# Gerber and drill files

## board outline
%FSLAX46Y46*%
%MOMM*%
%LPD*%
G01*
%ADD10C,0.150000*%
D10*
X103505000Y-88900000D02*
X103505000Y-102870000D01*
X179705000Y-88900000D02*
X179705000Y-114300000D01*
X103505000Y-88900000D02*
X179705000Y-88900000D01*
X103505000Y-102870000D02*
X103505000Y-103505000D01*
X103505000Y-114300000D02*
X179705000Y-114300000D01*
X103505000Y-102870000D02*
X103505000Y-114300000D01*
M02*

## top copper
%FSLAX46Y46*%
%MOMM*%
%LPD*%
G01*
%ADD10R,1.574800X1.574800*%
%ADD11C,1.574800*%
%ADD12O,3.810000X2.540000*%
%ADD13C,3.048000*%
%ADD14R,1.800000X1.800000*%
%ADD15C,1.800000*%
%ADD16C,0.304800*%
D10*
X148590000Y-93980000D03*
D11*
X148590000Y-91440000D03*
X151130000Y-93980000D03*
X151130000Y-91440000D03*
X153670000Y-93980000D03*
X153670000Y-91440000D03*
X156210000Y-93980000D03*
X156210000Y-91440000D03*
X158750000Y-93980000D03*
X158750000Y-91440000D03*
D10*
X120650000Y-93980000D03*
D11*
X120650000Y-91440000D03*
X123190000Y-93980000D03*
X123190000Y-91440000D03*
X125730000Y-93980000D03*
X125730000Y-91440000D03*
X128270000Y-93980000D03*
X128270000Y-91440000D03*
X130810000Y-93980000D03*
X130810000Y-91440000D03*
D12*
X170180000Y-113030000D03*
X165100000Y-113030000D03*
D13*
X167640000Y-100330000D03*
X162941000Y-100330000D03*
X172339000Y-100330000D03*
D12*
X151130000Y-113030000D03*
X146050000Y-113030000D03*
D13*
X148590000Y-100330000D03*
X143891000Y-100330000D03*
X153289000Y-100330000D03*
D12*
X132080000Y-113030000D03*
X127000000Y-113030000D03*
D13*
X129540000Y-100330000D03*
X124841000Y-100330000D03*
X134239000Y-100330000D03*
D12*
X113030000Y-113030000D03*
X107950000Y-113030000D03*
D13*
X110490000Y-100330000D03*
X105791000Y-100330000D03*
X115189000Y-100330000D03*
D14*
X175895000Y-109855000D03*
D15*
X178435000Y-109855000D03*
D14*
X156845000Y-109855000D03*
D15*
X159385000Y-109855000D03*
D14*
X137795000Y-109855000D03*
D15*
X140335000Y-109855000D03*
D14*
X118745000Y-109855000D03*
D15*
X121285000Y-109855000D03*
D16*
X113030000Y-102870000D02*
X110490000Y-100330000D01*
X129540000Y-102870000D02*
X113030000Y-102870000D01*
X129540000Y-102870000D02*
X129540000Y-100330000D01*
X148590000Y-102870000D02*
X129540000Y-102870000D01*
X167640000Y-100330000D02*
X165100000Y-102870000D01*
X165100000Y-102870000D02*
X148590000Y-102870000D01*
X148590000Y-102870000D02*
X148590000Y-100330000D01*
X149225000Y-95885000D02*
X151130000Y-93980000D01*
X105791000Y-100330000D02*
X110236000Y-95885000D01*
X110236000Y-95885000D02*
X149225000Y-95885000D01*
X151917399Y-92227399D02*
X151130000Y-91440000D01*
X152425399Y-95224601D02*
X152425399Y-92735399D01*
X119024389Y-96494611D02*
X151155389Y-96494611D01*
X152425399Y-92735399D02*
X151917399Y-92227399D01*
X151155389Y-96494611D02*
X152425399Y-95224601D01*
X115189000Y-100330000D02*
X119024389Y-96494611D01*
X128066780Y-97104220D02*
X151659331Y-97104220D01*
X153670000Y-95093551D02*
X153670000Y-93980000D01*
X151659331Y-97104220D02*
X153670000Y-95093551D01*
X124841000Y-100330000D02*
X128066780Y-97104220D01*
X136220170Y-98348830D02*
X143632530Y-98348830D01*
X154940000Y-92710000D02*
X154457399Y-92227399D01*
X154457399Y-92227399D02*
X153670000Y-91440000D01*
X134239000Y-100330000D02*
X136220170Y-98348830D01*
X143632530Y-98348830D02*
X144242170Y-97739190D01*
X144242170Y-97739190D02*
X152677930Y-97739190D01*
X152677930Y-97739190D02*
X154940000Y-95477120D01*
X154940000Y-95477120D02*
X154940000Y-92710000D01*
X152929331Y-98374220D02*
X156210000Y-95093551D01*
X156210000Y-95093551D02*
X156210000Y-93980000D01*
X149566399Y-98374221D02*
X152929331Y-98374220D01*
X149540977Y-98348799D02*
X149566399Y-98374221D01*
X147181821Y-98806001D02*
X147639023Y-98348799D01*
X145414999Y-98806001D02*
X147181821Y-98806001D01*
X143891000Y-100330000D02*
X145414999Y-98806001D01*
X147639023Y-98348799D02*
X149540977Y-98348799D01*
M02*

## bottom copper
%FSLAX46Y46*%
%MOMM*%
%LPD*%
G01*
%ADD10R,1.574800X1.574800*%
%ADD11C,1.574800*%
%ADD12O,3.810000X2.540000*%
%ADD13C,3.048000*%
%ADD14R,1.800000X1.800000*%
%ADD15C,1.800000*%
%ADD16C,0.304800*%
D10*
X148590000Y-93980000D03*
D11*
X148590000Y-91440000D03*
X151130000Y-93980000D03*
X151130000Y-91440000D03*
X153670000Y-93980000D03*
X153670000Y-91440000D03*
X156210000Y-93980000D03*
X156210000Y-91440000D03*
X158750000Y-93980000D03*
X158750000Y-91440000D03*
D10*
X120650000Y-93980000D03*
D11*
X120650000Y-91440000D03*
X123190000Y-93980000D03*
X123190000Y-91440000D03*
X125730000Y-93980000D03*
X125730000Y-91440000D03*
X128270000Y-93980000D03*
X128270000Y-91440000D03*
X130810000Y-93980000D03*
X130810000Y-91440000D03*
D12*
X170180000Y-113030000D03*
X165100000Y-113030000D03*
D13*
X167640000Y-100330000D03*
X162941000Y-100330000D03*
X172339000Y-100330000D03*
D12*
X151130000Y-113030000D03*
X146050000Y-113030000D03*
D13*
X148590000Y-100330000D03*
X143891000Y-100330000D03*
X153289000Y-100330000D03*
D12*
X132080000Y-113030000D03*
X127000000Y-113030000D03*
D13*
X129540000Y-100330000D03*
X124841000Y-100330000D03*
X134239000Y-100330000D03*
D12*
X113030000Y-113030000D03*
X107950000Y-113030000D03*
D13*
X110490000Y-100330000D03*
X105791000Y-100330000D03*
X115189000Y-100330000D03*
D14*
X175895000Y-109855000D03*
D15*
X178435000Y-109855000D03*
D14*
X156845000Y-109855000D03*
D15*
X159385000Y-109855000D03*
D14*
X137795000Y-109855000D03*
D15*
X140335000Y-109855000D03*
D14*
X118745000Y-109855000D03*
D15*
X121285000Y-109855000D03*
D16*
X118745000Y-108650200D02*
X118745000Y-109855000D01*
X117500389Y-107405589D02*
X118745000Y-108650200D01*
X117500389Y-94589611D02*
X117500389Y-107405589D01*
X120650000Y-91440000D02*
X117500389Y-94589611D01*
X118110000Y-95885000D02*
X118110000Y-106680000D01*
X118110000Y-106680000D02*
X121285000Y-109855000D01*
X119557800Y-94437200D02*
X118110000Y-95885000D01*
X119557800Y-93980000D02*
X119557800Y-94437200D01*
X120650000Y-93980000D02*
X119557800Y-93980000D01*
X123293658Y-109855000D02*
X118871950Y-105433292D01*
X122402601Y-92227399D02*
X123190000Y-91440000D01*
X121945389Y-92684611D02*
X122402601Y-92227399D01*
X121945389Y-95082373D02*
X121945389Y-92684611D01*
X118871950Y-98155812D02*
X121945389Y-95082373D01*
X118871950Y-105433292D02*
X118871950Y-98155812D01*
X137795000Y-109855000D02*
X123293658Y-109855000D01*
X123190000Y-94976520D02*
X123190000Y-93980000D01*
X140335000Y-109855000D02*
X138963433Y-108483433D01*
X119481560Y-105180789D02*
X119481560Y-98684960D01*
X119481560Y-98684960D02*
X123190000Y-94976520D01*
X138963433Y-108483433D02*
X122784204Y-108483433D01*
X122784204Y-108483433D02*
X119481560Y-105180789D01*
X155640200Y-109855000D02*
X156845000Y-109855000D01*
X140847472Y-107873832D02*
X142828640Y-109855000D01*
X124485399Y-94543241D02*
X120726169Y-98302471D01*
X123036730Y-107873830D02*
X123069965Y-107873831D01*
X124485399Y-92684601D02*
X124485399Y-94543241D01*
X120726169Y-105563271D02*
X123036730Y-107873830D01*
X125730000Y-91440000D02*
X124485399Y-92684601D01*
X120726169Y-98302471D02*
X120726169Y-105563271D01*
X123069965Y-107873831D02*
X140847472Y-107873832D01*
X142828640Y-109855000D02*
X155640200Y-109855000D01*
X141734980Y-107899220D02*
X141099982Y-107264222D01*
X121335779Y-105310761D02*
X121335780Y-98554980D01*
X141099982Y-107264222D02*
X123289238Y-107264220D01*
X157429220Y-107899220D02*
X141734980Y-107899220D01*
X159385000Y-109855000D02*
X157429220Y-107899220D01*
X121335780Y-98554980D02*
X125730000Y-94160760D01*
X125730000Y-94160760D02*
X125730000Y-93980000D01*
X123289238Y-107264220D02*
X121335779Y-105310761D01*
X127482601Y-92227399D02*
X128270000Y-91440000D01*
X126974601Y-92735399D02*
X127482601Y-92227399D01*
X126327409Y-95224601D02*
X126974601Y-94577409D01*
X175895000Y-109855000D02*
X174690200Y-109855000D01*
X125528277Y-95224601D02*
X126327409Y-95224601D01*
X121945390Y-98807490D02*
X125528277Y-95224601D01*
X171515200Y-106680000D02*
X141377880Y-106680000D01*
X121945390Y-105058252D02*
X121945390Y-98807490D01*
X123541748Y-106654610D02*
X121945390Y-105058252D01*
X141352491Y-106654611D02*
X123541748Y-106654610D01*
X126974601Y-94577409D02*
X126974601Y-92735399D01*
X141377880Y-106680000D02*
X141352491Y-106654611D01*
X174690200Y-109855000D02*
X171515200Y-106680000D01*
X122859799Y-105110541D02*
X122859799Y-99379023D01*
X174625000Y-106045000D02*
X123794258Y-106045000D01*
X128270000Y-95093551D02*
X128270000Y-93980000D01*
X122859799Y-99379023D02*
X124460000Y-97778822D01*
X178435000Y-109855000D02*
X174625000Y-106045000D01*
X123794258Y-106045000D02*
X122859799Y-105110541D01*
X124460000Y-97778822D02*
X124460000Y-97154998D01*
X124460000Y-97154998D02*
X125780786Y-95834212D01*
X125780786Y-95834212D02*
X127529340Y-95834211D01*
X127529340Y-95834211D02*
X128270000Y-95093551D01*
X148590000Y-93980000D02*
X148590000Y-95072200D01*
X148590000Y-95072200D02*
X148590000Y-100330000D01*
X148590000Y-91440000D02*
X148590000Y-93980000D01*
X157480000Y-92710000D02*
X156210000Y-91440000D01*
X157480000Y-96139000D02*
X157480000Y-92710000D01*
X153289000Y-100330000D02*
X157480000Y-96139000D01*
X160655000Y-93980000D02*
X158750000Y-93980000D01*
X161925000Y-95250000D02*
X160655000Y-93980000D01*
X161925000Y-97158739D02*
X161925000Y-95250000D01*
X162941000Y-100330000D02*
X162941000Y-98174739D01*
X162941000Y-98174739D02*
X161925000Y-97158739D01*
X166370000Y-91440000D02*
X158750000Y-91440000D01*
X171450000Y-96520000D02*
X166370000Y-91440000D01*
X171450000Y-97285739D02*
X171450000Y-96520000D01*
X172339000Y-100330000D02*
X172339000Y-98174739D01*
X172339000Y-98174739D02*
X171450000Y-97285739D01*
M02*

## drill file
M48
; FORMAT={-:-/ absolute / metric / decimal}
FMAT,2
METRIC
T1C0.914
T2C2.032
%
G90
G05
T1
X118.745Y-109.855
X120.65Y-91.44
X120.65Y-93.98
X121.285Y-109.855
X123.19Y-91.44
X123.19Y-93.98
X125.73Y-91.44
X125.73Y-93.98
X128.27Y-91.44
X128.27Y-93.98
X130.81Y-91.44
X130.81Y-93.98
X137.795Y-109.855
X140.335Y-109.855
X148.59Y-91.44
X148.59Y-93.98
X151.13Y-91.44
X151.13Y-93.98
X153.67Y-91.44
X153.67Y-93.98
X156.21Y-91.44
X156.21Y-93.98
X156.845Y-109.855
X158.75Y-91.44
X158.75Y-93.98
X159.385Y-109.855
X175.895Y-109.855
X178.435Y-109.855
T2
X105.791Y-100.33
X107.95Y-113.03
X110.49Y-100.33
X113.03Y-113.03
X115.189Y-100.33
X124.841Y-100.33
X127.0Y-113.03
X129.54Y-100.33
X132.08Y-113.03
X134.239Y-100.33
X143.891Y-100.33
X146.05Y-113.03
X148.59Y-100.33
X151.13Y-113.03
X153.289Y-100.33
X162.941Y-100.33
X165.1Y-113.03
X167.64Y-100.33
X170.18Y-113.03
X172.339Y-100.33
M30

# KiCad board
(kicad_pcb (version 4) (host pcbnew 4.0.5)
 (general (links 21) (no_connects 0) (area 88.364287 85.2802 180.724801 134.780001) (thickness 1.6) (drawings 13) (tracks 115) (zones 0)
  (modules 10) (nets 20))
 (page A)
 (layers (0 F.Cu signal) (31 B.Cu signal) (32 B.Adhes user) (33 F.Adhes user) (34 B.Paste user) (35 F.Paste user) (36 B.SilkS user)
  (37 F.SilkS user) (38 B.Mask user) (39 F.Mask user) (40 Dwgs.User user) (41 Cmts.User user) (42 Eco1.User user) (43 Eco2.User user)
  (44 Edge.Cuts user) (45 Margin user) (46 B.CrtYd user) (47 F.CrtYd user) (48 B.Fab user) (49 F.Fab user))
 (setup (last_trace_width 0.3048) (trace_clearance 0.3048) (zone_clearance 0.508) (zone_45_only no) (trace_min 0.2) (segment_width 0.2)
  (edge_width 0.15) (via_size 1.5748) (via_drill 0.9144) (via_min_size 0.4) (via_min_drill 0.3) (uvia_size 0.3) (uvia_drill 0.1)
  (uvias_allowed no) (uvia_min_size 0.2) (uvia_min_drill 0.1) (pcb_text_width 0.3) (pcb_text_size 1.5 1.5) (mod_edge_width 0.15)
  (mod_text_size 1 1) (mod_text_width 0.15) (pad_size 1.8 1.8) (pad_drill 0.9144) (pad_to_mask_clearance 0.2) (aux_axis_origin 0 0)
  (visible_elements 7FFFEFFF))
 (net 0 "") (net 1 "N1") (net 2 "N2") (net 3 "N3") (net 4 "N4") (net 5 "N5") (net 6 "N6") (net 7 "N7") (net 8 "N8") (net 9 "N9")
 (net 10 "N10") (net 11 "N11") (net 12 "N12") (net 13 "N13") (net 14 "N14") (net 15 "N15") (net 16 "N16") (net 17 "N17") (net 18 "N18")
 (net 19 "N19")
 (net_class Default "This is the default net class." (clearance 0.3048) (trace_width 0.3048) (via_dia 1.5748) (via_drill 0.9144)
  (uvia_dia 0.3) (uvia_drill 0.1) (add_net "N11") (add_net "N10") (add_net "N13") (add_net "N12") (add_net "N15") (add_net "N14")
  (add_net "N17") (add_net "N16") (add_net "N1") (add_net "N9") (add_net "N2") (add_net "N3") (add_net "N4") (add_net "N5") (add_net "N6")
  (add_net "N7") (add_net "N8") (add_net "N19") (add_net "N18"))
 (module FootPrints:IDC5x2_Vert (layer F.Cu) (at 153.67 92.71 180)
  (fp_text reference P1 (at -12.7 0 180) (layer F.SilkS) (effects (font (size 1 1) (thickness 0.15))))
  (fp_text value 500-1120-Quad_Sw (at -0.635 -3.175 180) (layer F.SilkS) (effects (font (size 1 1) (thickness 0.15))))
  (pad 1 thru_hole rect (at 5.08 -1.27 180) (size 1.5748 1.5748) (drill 0.9144) (layers *.Cu *.Mask F.SilkS) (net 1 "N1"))
  (pad 2 thru_hole circle (at 5.08 1.27 180) (size 1.5748 1.5748) (drill 0.9144) (layers *.Cu *.Mask F.SilkS) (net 1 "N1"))
  (pad 3 thru_hole circle (at 2.54 -1.27 180) (size 1.5748 1.5748) (drill 0.9144) (layers *.Cu *.Mask F.SilkS) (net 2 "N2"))
  (pad 4 thru_hole circle (at 2.54 1.27 180) (size 1.5748 1.5748) (drill 0.9144) (layers *.Cu *.Mask F.SilkS) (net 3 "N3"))
  (pad 5 thru_hole circle (at 0 -1.27 180) (size 1.5748 1.5748) (drill 0.9144) (layers *.Cu *.Mask F.SilkS) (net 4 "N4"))
  (pad 6 thru_hole circle (at 0 1.27 180) (size 1.5748 1.5748) (drill 0.9144) (layers *.Cu *.Mask F.SilkS) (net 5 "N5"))
  (pad 7 thru_hole circle (at -2.54 -1.27 180) (size 1.5748 1.5748) (drill 0.9144) (layers *.Cu *.Mask F.SilkS) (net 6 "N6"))
  (pad 8 thru_hole circle (at -2.54 1.27 180) (size 1.5748 1.5748) (drill 0.9144) (layers *.Cu *.Mask F.SilkS) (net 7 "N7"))
  (pad 9 thru_hole circle (at -5.08 -1.27 180) (size 1.5748 1.5748) (drill 0.9144) (layers *.Cu *.Mask F.SilkS) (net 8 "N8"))
  (pad 10 thru_hole circle (at -5.08 1.27 180) (size 1.5748 1.5748) (drill 0.9144) (layers *.Cu *.Mask F.SilkS) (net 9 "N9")))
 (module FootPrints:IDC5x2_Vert (layer F.Cu) (at 125.73 92.71 180)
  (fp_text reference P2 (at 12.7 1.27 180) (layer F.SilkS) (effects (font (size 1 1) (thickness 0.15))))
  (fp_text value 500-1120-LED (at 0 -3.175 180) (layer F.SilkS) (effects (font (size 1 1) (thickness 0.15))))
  (pad 1 thru_hole rect (at 5.08 -1.27 180) (size 1.5748 1.5748) (drill 0.9144) (layers *.Cu *.Mask F.SilkS) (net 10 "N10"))
  (pad 2 thru_hole circle (at 5.08 1.27 180) (size 1.5748 1.5748) (drill 0.9144) (layers *.Cu *.Mask F.SilkS) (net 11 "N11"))
  (pad 3 thru_hole circle (at 2.54 -1.27 180) (size 1.5748 1.5748) (drill 0.9144) (layers *.Cu *.Mask F.SilkS) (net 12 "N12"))
  (pad 4 thru_hole circle (at 2.54 1.27 180) (size 1.5748 1.5748) (drill 0.9144) (layers *.Cu *.Mask F.SilkS) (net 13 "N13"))
  (pad 5 thru_hole circle (at 0 -1.27 180) (size 1.5748 1.5748) (drill 0.9144) (layers *.Cu *.Mask F.SilkS) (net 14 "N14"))
  (pad 6 thru_hole circle (at 0 1.27 180) (size 1.5748 1.5748) (drill 0.9144) (layers *.Cu *.Mask F.SilkS) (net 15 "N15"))
  (pad 7 thru_hole circle (at -2.54 -1.27 180) (size 1.5748 1.5748) (drill 0.9144) (layers *.Cu *.Mask F.SilkS) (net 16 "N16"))
  (pad 8 thru_hole circle (at -2.54 1.27 180) (size 1.5748 1.5748) (drill 0.9144) (layers *.Cu *.Mask F.SilkS) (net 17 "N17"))
  (pad 9 thru_hole circle (at -5.08 -1.27 180) (size 1.5748 1.5748) (drill 0.9144) (layers *.Cu *.Mask F.SilkS) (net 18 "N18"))
  (pad 10 thru_hole circle (at -5.08 1.27 180) (size 1.5748 1.5748) (drill 0.9144) (layers *.Cu *.Mask F.SilkS) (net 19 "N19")))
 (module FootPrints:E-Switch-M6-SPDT (layer F.Cu) (at 167.64 113.03 180)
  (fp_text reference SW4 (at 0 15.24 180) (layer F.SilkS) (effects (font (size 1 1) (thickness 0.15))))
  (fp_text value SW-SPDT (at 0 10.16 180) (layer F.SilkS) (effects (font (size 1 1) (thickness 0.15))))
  (pad 4 thru_hole oval (at -2.54 0 180) (size 3.81 2.54) (drill 2.032) (layers *.Cu *.Mask))
  (pad 5 thru_hole oval (at 2.54 0 180) (size 3.81 2.54) (drill 2.032) (layers *.Cu *.Mask))
  (pad 2 thru_hole circle (at 0 12.7 180) (size 3.048 3.048) (drill 2.032) (layers *.Cu *.Mask) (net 1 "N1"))
  (pad 3 thru_hole circle (at 4.699 12.7 180) (size 3.048 3.048) (drill 2.032) (layers *.Cu *.Mask) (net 8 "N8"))
  (pad 1 thru_hole circle (at -4.699 12.7 180) (size 3.048 3.048) (drill 2.032) (layers *.Cu *.Mask) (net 9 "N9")))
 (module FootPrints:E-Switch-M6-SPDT (layer F.Cu) (at 148.59 113.03 180)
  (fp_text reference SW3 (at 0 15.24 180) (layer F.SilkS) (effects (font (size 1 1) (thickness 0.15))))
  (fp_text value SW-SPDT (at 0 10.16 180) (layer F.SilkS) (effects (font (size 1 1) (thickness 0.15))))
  (pad 4 thru_hole oval (at -2.54 0 180) (size 3.81 2.54) (drill 2.032) (layers *.Cu *.Mask))
  (pad 5 thru_hole oval (at 2.54 0 180) (size 3.81 2.54) (drill 2.032) (layers *.Cu *.Mask))
  (pad 2 thru_hole circle (at 0 12.7 180) (size 3.048 3.048) (drill 2.032) (layers *.Cu *.Mask) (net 1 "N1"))
  (pad 3 thru_hole circle (at 4.699 12.7 180) (size 3.048 3.048) (drill 2.032) (layers *.Cu *.Mask) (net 6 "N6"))
  (pad 1 thru_hole circle (at -4.699 12.7 180) (size 3.048 3.048) (drill 2.032) (layers *.Cu *.Mask) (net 7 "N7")))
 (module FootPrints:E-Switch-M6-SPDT (layer F.Cu) (at 129.54 113.03 180)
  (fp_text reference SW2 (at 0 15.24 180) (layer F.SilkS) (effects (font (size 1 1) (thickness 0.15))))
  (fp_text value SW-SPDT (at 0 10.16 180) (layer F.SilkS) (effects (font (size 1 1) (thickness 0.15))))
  (pad 4 thru_hole oval (at -2.54 0 180) (size 3.81 2.54) (drill 2.032) (layers *.Cu *.Mask))
  (pad 5 thru_hole oval (at 2.54 0 180) (size 3.81 2.54) (drill 2.032) (layers *.Cu *.Mask))
  (pad 2 thru_hole circle (at 0 12.7 180) (size 3.048 3.048) (drill 2.032) (layers *.Cu *.Mask) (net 1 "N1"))
  (pad 3 thru_hole circle (at 4.699 12.7 180) (size 3.048 3.048) (drill 2.032) (layers *.Cu *.Mask) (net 4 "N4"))
  (pad 1 thru_hole circle (at -4.699 12.7 180) (size 3.048 3.048) (drill 2.032) (layers *.Cu *.Mask) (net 5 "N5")))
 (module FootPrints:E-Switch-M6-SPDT (layer F.Cu) (at 110.49 113.03 180)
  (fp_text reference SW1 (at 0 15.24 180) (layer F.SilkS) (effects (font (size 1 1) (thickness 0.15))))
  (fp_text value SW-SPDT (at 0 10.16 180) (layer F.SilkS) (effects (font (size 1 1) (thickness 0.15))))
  (pad 4 thru_hole oval (at -2.54 0 180) (size 3.81 2.54) (drill 2.032) (layers *.Cu *.Mask))
  (pad 5 thru_hole oval (at 2.54 0 180) (size 3.81 2.54) (drill 2.032) (layers *.Cu *.Mask))
  (pad 2 thru_hole circle (at 0 12.7 180) (size 3.048 3.048) (drill 2.032) (layers *.Cu *.Mask) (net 1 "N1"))
  (pad 3 thru_hole circle (at 4.699 12.7 180) (size 3.048 3.048) (drill 2.032) (layers *.Cu *.Mask) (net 2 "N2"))
  (pad 1 thru_hole circle (at -4.699 12.7 180) (size 3.048 3.048) (drill 2.032) (layers *.Cu *.Mask) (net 3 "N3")))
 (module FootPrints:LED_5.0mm (layer F.Cu) (at 175.895 109.855)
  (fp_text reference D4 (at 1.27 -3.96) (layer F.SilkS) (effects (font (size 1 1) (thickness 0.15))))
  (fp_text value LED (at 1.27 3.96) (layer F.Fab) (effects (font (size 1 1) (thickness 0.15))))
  (pad 1 thru_hole rect (at 0 0) (size 1.8 1.8) (drill 0.9144) (layers *.Cu *.Mask) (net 17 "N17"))
  (pad 2 thru_hole circle (at 2.54 0) (size 1.8 1.8) (drill 0.9144) (layers *.Cu *.Mask) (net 16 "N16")))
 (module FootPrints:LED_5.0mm (layer F.Cu) (at 156.845 109.855)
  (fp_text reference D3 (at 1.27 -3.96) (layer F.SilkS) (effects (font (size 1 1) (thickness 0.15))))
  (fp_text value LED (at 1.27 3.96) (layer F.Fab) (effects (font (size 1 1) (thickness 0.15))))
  (pad 1 thru_hole rect (at 0 0) (size 1.8 1.8) (drill 0.9144) (layers *.Cu *.Mask) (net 15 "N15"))
  (pad 2 thru_hole circle (at 2.54 0) (size 1.8 1.8) (drill 0.9144) (layers *.Cu *.Mask) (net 14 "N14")))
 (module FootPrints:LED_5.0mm (layer F.Cu) (at 137.795 109.855)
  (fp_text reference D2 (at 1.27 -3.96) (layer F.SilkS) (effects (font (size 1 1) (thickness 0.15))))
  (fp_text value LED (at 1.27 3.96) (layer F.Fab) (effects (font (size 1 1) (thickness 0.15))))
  (pad 1 thru_hole rect (at 0 0) (size 1.8 1.8) (drill 0.9144) (layers *.Cu *.Mask) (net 13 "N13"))
  (pad 2 thru_hole circle (at 2.54 0) (size 1.8 1.8) (drill 0.9144) (layers *.Cu *.Mask) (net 12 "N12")))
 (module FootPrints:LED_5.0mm (layer F.Cu) (at 118.745 109.855)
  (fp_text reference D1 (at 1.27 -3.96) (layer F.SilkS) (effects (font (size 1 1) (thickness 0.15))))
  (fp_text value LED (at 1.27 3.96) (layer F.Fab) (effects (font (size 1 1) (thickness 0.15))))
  (pad 1 thru_hole rect (at 0 0) (size 1.8 1.8) (drill 0.9144) (layers *.Cu *.Mask) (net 11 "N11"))
  (pad 2 thru_hole circle (at 2.54 0) (size 1.8 1.8) (drill 0.9144) (layers *.Cu *.Mask) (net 10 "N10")))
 (gr_line (start 103.505 88.9) (end 103.505 102.87) (angle 90) (layer Edge.Cuts) (width 0.15))
 (gr_line (start 179.705 88.9) (end 179.705 114.3) (angle 90) (layer Edge.Cuts) (width 0.15))
 (gr_line (start 103.505 88.9) (end 179.705 88.9) (angle 90) (layer Edge.Cuts) (width 0.15))
 (gr_line (start 103.505 102.87) (end 103.505 103.505) (angle 90) (layer Edge.Cuts) (width 0.15))
 (gr_line (start 103.505 114.3) (end 179.705 114.3) (angle 90) (layer Edge.Cuts) (width 0.15))
 (gr_line (start 103.505 102.87) (end 103.505 114.3) (angle 90) (layer Edge.Cuts) (width 0.15))
 (segment (start 118.745 108.6502) (end 118.745 109.855) (width 0.3048) (layer B.Cu) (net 11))
 (segment (start 117.500389 107.405589) (end 118.745 108.6502) (width 0.3048) (layer B.Cu) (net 11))
 (segment (start 117.500389 94.589611) (end 117.500389 107.405589) (width 0.3048) (layer B.Cu) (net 11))
 (segment (start 120.65 91.44) (end 117.500389 94.589611) (width 0.3048) (layer B.Cu) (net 11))
 (segment (start 118.11 95.885) (end 118.11 106.68) (width 0.3048) (layer B.Cu) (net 10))
 (segment (start 118.11 106.68) (end 121.285 109.855) (width 0.3048) (layer B.Cu) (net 10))
 (segment (start 119.5578 94.4372) (end 118.11 95.885) (width 0.3048) (layer B.Cu) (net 10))
 (segment (start 119.5578 93.98) (end 119.5578 94.4372) (width 0.3048) (layer B.Cu) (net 10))
 (segment (start 120.65 93.98) (end 119.5578 93.98) (width 0.3048) (layer B.Cu) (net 10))
 (segment (start 123.293658 109.855) (end 118.87195 105.433292) (width 0.3048) (layer B.Cu) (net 13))
 (segment (start 122.402601 92.227399) (end 123.19 91.44) (width 0.3048) (layer B.Cu) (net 13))
 (segment (start 121.945389 92.684611) (end 122.402601 92.227399) (width 0.3048) (layer B.Cu) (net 13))
 (segment (start 121.945389 95.082373) (end 121.945389 92.684611) (width 0.3048) (layer B.Cu) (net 13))
 (segment (start 118.87195 98.155812) (end 121.945389 95.082373) (width 0.3048) (layer B.Cu) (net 13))
 (segment (start 118.87195 105.433292) (end 118.87195 98.155812) (width 0.3048) (layer B.Cu) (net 13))
 (segment (start 137.795 109.855) (end 123.293658 109.855) (width 0.3048) (layer B.Cu) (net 13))
 (segment (start 123.19 94.97652) (end 123.19 93.98) (width 0.3048) (layer B.Cu) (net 12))
 (segment (start 140.335 109.855) (end 138.963433 108.483433) (width 0.3048) (layer B.Cu) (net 12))
 (segment (start 119.48156 105.180789) (end 119.48156 98.68496) (width 0.3048) (layer B.Cu) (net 12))
 (segment (start 119.48156 98.68496) (end 123.19 94.97652) (width 0.3048) (layer B.Cu) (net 12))
 (segment (start 138.963433 108.483433) (end 122.784204 108.483433) (width 0.3048) (layer B.Cu) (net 12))
 (segment (start 122.784204 108.483433) (end 119.48156 105.180789) (width 0.3048) (layer B.Cu) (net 12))
 (segment (start 155.6402 109.855) (end 156.845 109.855) (width 0.3048) (layer B.Cu) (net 15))
 (segment (start 140.847472 107.873832) (end 142.82864 109.855) (width 0.3048) (layer B.Cu) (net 15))
 (segment (start 124.485399 94.543241) (end 120.726169 98.302471) (width 0.3048) (layer B.Cu) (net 15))
 (segment (start 123.03673 107.87383) (end 123.069965 107.873831) (width 0.3048) (layer B.Cu) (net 15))
 (segment (start 124.485399 92.684601) (end 124.485399 94.543241) (width 0.3048) (layer B.Cu) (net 15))
 (segment (start 120.726169 105.563271) (end 123.03673 107.87383) (width 0.3048) (layer B.Cu) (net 15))
 (segment (start 125.73 91.44) (end 124.485399 92.684601) (width 0.3048) (layer B.Cu) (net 15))
 (segment (start 120.726169 98.302471) (end 120.726169 105.563271) (width 0.3048) (layer B.Cu) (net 15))
 (segment (start 123.069965 107.873831) (end 140.847472 107.873832) (width 0.3048) (layer B.Cu) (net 15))
 (segment (start 142.82864 109.855) (end 155.6402 109.855) (width 0.3048) (layer B.Cu) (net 15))
 (segment (start 141.73498 107.89922) (end 141.099982 107.264222) (width 0.3048) (layer B.Cu) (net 14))
 (segment (start 121.335779 105.310761) (end 121.33578 98.55498) (width 0.3048) (layer B.Cu) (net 14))
 (segment (start 141.099982 107.264222) (end 123.289238 107.26422) (width 0.3048) (layer B.Cu) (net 14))
 (segment (start 157.42922 107.89922) (end 141.73498 107.89922) (width 0.3048) (layer B.Cu) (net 14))
 (segment (start 159.385 109.855) (end 157.42922 107.89922) (width 0.3048) (layer B.Cu) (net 14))
 (segment (start 121.33578 98.55498) (end 125.73 94.16076) (width 0.3048) (layer B.Cu) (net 14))
 (segment (start 125.73 94.16076) (end 125.73 93.98) (width 0.3048) (layer B.Cu) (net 14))
 (segment (start 123.289238 107.26422) (end 121.335779 105.310761) (width 0.3048) (layer B.Cu) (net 14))
 (segment (start 127.482601 92.227399) (end 128.27 91.44) (width 0.3048) (layer B.Cu) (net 17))
 (segment (start 126.974601 92.735399) (end 127.482601 92.227399) (width 0.3048) (layer B.Cu) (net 17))
 (segment (start 126.327409 95.224601) (end 126.974601 94.577409) (width 0.3048) (layer B.Cu) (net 17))
 (segment (start 175.895 109.855) (end 174.6902 109.855) (width 0.3048) (layer B.Cu) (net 17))
 (segment (start 125.528277 95.224601) (end 126.327409 95.224601) (width 0.3048) (layer B.Cu) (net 17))
 (segment (start 121.94539 98.80749) (end 125.528277 95.224601) (width 0.3048) (layer B.Cu) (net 17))
 (segment (start 171.5152 106.68) (end 141.37788 106.68) (width 0.3048) (layer B.Cu) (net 17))
 (segment (start 121.94539 105.058252) (end 121.94539 98.80749) (width 0.3048) (layer B.Cu) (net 17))
 (segment (start 123.541748 106.65461) (end 121.94539 105.058252) (width 0.3048) (layer B.Cu) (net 17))
 (segment (start 141.352491 106.654611) (end 123.541748 106.65461) (width 0.3048) (layer B.Cu) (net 17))
 (segment (start 126.974601 94.577409) (end 126.974601 92.735399) (width 0.3048) (layer B.Cu) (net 17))
 (segment (start 141.37788 106.68) (end 141.352491 106.654611) (width 0.3048) (layer B.Cu) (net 17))
 (segment (start 174.6902 109.855) (end 171.5152 106.68) (width 0.3048) (layer B.Cu) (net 17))
 (segment (start 122.859799 105.110541) (end 122.859799 99.379023) (width 0.3048) (layer B.Cu) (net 16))
 (segment (start 174.625 106.045) (end 123.794258 106.045) (width 0.3048) (layer B.Cu) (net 16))
 (segment (start 128.27 95.093551) (end 128.27 93.98) (width 0.3048) (layer B.Cu) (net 16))
 (segment (start 122.859799 99.379023) (end 124.46 97.778822) (width 0.3048) (layer B.Cu) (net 16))
 (segment (start 178.435 109.855) (end 174.625 106.045) (width 0.3048) (layer B.Cu) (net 16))
 (segment (start 123.794258 106.045) (end 122.859799 105.110541) (width 0.3048) (layer B.Cu) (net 16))
 (segment (start 124.46 97.778822) (end 124.46 97.154998) (width 0.3048) (layer B.Cu) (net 16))
 (segment (start 124.46 97.154998) (end 125.780786 95.834212) (width 0.3048) (layer B.Cu) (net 16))
 (segment (start 125.780786 95.834212) (end 127.52934 95.834211) (width 0.3048) (layer B.Cu) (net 16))
 (segment (start 127.52934 95.834211) (end 128.27 95.093551) (width 0.3048) (layer B.Cu) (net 16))
 (segment (start 148.59 93.98) (end 148.59 95.0722) (width 0.3048) (layer B.Cu) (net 1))
 (segment (start 148.59 95.0722) (end 148.59 100.33) (width 0.3048) (layer B.Cu) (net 1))
 (segment (start 148.59 91.44) (end 148.59 93.98) (width 0.3048) (layer B.Cu) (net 1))
 (segment (start 113.03 102.87) (end 110.49 100.33) (width 0.3048) (layer F.Cu) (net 1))
 (segment (start 129.54 102.87) (end 113.03 102.87) (width 0.3048) (layer F.Cu) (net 1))
 (segment (start 129.54 102.87) (end 129.54 100.33) (width 0.3048) (layer F.Cu) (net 1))
 (segment (start 148.59 102.87) (end 129.54 102.87) (width 0.3048) (layer F.Cu) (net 1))
 (segment (start 167.64 100.33) (end 165.1 102.87) (width 0.3048) (layer F.Cu) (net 1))
 (segment (start 165.1 102.87) (end 148.59 102.87) (width 0.3048) (layer F.Cu) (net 1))
 (segment (start 148.59 102.87) (end 148.59 100.33) (width 0.3048) (layer F.Cu) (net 1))
 (segment (start 149.225 95.885) (end 151.13 93.98) (width 0.3048) (layer F.Cu) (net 2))
 (segment (start 105.791 100.33) (end 110.236 95.885) (width 0.3048) (layer F.Cu) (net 2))
 (segment (start 110.236 95.885) (end 149.225 95.885) (width 0.3048) (layer F.Cu) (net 2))
 (segment (start 151.917399 92.227399) (end 151.13 91.44) (width 0.3048) (layer F.Cu) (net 3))
 (segment (start 152.425399 95.224601) (end 152.425399 92.735399) (width 0.3048) (layer F.Cu) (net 3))
 (segment (start 119.024389 96.494611) (end 151.155389 96.494611) (width 0.3048) (layer F.Cu) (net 3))
 (segment (start 152.425399 92.735399) (end 151.917399 92.227399) (width 0.3048) (layer F.Cu) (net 3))
 (segment (start 151.155389 96.494611) (end 152.425399 95.224601) (width 0.3048) (layer F.Cu) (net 3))
 (segment (start 115.189 100.33) (end 119.024389 96.494611) (width 0.3048) (layer F.Cu) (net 3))
 (segment (start 128.06678 97.10422) (end 151.659331 97.10422) (width 0.3048) (layer F.Cu) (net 4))
 (segment (start 153.67 95.093551) (end 153.67 93.98) (width 0.3048) (layer F.Cu) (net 4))
 (segment (start 151.659331 97.10422) (end 153.67 95.093551) (width 0.3048) (layer F.Cu) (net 4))
 (segment (start 124.841 100.33) (end 128.06678 97.10422) (width 0.3048) (layer F.Cu) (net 4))
 (segment (start 136.22017 98.34883) (end 143.63253 98.34883) (width 0.3048) (layer F.Cu) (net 5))
 (segment (start 154.94 92.71) (end 154.457399 92.227399) (width 0.3048) (layer F.Cu) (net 5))
 (segment (start 154.457399 92.227399) (end 153.67 91.44) (width 0.3048) (layer F.Cu) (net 5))
 (segment (start 134.239 100.33) (end 136.22017 98.34883) (width 0.3048) (layer F.Cu) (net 5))
 (segment (start 143.63253 98.34883) (end 144.24217 97.73919) (width 0.3048) (layer F.Cu) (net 5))
 (segment (start 144.24217 97.73919) (end 152.67793 97.73919) (width 0.3048) (layer F.Cu) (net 5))
 (segment (start 152.67793 97.73919) (end 154.94 95.47712) (width 0.3048) (layer F.Cu) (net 5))
 (segment (start 154.94 95.47712) (end 154.94 92.71) (width 0.3048) (layer F.Cu) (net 5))
 (segment (start 152.929331 98.37422) (end 156.21 95.093551) (width 0.3048) (layer F.Cu) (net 6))
 (segment (start 156.21 95.093551) (end 156.21 93.98) (width 0.3048) (layer F.Cu) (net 6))
 (segment (start 149.566399 98.374221) (end 152.929331 98.37422) (width 0.3048) (layer F.Cu) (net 6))
 (segment (start 149.540977 98.348799) (end 149.566399 98.374221) (width 0.3048) (layer F.Cu) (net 6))
 (segment (start 147.181821 98.806001) (end 147.639023 98.348799) (width 0.3048) (layer F.Cu) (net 6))
 (segment (start 145.414999 98.806001) (end 147.181821 98.806001) (width 0.3048) (layer F.Cu) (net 6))
 (segment (start 143.891 100.33) (end 145.414999 98.806001) (width 0.3048) (layer F.Cu) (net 6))
 (segment (start 147.639023 98.348799) (end 149.540977 98.348799) (width 0.3048) (layer F.Cu) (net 6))
 (segment (start 157.48 92.71) (end 156.21 91.44) (width 0.3048) (layer B.Cu) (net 7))
 (segment (start 157.48 96.139) (end 157.48 92.71) (width 0.3048) (layer B.Cu) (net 7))
 (segment (start 153.289 100.33) (end 157.48 96.139) (width 0.3048) (layer B.Cu) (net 7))
 (segment (start 160.655 93.98) (end 158.75 93.98) (width 0.3048) (layer B.Cu) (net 8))
 (segment (start 161.925 95.25) (end 160.655 93.98) (width 0.3048) (layer B.Cu) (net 8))
 (segment (start 161.925 97.158739) (end 161.925 95.25) (width 0.3048) (layer B.Cu) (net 8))
 (segment (start 162.941 100.33) (end 162.941 98.174739) (width 0.3048) (layer B.Cu) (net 8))
 (segment (start 162.941 98.174739) (end 161.925 97.158739) (width 0.3048) (layer B.Cu) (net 8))
 (segment (start 166.37 91.44) (end 158.75 91.44) (width 0.3048) (layer B.Cu) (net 9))
 (segment (start 171.45 96.52) (end 166.37 91.44) (width 0.3048) (layer B.Cu) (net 9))
 (segment (start 171.45 97.285739) (end 171.45 96.52) (width 0.3048) (layer B.Cu) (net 9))
 (segment (start 172.339 100.33) (end 172.339 98.174739) (width 0.3048) (layer B.Cu) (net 9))
 (segment (start 172.339 98.174739) (end 171.45 97.285739) (width 0.3048) (layer B.Cu) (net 9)))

